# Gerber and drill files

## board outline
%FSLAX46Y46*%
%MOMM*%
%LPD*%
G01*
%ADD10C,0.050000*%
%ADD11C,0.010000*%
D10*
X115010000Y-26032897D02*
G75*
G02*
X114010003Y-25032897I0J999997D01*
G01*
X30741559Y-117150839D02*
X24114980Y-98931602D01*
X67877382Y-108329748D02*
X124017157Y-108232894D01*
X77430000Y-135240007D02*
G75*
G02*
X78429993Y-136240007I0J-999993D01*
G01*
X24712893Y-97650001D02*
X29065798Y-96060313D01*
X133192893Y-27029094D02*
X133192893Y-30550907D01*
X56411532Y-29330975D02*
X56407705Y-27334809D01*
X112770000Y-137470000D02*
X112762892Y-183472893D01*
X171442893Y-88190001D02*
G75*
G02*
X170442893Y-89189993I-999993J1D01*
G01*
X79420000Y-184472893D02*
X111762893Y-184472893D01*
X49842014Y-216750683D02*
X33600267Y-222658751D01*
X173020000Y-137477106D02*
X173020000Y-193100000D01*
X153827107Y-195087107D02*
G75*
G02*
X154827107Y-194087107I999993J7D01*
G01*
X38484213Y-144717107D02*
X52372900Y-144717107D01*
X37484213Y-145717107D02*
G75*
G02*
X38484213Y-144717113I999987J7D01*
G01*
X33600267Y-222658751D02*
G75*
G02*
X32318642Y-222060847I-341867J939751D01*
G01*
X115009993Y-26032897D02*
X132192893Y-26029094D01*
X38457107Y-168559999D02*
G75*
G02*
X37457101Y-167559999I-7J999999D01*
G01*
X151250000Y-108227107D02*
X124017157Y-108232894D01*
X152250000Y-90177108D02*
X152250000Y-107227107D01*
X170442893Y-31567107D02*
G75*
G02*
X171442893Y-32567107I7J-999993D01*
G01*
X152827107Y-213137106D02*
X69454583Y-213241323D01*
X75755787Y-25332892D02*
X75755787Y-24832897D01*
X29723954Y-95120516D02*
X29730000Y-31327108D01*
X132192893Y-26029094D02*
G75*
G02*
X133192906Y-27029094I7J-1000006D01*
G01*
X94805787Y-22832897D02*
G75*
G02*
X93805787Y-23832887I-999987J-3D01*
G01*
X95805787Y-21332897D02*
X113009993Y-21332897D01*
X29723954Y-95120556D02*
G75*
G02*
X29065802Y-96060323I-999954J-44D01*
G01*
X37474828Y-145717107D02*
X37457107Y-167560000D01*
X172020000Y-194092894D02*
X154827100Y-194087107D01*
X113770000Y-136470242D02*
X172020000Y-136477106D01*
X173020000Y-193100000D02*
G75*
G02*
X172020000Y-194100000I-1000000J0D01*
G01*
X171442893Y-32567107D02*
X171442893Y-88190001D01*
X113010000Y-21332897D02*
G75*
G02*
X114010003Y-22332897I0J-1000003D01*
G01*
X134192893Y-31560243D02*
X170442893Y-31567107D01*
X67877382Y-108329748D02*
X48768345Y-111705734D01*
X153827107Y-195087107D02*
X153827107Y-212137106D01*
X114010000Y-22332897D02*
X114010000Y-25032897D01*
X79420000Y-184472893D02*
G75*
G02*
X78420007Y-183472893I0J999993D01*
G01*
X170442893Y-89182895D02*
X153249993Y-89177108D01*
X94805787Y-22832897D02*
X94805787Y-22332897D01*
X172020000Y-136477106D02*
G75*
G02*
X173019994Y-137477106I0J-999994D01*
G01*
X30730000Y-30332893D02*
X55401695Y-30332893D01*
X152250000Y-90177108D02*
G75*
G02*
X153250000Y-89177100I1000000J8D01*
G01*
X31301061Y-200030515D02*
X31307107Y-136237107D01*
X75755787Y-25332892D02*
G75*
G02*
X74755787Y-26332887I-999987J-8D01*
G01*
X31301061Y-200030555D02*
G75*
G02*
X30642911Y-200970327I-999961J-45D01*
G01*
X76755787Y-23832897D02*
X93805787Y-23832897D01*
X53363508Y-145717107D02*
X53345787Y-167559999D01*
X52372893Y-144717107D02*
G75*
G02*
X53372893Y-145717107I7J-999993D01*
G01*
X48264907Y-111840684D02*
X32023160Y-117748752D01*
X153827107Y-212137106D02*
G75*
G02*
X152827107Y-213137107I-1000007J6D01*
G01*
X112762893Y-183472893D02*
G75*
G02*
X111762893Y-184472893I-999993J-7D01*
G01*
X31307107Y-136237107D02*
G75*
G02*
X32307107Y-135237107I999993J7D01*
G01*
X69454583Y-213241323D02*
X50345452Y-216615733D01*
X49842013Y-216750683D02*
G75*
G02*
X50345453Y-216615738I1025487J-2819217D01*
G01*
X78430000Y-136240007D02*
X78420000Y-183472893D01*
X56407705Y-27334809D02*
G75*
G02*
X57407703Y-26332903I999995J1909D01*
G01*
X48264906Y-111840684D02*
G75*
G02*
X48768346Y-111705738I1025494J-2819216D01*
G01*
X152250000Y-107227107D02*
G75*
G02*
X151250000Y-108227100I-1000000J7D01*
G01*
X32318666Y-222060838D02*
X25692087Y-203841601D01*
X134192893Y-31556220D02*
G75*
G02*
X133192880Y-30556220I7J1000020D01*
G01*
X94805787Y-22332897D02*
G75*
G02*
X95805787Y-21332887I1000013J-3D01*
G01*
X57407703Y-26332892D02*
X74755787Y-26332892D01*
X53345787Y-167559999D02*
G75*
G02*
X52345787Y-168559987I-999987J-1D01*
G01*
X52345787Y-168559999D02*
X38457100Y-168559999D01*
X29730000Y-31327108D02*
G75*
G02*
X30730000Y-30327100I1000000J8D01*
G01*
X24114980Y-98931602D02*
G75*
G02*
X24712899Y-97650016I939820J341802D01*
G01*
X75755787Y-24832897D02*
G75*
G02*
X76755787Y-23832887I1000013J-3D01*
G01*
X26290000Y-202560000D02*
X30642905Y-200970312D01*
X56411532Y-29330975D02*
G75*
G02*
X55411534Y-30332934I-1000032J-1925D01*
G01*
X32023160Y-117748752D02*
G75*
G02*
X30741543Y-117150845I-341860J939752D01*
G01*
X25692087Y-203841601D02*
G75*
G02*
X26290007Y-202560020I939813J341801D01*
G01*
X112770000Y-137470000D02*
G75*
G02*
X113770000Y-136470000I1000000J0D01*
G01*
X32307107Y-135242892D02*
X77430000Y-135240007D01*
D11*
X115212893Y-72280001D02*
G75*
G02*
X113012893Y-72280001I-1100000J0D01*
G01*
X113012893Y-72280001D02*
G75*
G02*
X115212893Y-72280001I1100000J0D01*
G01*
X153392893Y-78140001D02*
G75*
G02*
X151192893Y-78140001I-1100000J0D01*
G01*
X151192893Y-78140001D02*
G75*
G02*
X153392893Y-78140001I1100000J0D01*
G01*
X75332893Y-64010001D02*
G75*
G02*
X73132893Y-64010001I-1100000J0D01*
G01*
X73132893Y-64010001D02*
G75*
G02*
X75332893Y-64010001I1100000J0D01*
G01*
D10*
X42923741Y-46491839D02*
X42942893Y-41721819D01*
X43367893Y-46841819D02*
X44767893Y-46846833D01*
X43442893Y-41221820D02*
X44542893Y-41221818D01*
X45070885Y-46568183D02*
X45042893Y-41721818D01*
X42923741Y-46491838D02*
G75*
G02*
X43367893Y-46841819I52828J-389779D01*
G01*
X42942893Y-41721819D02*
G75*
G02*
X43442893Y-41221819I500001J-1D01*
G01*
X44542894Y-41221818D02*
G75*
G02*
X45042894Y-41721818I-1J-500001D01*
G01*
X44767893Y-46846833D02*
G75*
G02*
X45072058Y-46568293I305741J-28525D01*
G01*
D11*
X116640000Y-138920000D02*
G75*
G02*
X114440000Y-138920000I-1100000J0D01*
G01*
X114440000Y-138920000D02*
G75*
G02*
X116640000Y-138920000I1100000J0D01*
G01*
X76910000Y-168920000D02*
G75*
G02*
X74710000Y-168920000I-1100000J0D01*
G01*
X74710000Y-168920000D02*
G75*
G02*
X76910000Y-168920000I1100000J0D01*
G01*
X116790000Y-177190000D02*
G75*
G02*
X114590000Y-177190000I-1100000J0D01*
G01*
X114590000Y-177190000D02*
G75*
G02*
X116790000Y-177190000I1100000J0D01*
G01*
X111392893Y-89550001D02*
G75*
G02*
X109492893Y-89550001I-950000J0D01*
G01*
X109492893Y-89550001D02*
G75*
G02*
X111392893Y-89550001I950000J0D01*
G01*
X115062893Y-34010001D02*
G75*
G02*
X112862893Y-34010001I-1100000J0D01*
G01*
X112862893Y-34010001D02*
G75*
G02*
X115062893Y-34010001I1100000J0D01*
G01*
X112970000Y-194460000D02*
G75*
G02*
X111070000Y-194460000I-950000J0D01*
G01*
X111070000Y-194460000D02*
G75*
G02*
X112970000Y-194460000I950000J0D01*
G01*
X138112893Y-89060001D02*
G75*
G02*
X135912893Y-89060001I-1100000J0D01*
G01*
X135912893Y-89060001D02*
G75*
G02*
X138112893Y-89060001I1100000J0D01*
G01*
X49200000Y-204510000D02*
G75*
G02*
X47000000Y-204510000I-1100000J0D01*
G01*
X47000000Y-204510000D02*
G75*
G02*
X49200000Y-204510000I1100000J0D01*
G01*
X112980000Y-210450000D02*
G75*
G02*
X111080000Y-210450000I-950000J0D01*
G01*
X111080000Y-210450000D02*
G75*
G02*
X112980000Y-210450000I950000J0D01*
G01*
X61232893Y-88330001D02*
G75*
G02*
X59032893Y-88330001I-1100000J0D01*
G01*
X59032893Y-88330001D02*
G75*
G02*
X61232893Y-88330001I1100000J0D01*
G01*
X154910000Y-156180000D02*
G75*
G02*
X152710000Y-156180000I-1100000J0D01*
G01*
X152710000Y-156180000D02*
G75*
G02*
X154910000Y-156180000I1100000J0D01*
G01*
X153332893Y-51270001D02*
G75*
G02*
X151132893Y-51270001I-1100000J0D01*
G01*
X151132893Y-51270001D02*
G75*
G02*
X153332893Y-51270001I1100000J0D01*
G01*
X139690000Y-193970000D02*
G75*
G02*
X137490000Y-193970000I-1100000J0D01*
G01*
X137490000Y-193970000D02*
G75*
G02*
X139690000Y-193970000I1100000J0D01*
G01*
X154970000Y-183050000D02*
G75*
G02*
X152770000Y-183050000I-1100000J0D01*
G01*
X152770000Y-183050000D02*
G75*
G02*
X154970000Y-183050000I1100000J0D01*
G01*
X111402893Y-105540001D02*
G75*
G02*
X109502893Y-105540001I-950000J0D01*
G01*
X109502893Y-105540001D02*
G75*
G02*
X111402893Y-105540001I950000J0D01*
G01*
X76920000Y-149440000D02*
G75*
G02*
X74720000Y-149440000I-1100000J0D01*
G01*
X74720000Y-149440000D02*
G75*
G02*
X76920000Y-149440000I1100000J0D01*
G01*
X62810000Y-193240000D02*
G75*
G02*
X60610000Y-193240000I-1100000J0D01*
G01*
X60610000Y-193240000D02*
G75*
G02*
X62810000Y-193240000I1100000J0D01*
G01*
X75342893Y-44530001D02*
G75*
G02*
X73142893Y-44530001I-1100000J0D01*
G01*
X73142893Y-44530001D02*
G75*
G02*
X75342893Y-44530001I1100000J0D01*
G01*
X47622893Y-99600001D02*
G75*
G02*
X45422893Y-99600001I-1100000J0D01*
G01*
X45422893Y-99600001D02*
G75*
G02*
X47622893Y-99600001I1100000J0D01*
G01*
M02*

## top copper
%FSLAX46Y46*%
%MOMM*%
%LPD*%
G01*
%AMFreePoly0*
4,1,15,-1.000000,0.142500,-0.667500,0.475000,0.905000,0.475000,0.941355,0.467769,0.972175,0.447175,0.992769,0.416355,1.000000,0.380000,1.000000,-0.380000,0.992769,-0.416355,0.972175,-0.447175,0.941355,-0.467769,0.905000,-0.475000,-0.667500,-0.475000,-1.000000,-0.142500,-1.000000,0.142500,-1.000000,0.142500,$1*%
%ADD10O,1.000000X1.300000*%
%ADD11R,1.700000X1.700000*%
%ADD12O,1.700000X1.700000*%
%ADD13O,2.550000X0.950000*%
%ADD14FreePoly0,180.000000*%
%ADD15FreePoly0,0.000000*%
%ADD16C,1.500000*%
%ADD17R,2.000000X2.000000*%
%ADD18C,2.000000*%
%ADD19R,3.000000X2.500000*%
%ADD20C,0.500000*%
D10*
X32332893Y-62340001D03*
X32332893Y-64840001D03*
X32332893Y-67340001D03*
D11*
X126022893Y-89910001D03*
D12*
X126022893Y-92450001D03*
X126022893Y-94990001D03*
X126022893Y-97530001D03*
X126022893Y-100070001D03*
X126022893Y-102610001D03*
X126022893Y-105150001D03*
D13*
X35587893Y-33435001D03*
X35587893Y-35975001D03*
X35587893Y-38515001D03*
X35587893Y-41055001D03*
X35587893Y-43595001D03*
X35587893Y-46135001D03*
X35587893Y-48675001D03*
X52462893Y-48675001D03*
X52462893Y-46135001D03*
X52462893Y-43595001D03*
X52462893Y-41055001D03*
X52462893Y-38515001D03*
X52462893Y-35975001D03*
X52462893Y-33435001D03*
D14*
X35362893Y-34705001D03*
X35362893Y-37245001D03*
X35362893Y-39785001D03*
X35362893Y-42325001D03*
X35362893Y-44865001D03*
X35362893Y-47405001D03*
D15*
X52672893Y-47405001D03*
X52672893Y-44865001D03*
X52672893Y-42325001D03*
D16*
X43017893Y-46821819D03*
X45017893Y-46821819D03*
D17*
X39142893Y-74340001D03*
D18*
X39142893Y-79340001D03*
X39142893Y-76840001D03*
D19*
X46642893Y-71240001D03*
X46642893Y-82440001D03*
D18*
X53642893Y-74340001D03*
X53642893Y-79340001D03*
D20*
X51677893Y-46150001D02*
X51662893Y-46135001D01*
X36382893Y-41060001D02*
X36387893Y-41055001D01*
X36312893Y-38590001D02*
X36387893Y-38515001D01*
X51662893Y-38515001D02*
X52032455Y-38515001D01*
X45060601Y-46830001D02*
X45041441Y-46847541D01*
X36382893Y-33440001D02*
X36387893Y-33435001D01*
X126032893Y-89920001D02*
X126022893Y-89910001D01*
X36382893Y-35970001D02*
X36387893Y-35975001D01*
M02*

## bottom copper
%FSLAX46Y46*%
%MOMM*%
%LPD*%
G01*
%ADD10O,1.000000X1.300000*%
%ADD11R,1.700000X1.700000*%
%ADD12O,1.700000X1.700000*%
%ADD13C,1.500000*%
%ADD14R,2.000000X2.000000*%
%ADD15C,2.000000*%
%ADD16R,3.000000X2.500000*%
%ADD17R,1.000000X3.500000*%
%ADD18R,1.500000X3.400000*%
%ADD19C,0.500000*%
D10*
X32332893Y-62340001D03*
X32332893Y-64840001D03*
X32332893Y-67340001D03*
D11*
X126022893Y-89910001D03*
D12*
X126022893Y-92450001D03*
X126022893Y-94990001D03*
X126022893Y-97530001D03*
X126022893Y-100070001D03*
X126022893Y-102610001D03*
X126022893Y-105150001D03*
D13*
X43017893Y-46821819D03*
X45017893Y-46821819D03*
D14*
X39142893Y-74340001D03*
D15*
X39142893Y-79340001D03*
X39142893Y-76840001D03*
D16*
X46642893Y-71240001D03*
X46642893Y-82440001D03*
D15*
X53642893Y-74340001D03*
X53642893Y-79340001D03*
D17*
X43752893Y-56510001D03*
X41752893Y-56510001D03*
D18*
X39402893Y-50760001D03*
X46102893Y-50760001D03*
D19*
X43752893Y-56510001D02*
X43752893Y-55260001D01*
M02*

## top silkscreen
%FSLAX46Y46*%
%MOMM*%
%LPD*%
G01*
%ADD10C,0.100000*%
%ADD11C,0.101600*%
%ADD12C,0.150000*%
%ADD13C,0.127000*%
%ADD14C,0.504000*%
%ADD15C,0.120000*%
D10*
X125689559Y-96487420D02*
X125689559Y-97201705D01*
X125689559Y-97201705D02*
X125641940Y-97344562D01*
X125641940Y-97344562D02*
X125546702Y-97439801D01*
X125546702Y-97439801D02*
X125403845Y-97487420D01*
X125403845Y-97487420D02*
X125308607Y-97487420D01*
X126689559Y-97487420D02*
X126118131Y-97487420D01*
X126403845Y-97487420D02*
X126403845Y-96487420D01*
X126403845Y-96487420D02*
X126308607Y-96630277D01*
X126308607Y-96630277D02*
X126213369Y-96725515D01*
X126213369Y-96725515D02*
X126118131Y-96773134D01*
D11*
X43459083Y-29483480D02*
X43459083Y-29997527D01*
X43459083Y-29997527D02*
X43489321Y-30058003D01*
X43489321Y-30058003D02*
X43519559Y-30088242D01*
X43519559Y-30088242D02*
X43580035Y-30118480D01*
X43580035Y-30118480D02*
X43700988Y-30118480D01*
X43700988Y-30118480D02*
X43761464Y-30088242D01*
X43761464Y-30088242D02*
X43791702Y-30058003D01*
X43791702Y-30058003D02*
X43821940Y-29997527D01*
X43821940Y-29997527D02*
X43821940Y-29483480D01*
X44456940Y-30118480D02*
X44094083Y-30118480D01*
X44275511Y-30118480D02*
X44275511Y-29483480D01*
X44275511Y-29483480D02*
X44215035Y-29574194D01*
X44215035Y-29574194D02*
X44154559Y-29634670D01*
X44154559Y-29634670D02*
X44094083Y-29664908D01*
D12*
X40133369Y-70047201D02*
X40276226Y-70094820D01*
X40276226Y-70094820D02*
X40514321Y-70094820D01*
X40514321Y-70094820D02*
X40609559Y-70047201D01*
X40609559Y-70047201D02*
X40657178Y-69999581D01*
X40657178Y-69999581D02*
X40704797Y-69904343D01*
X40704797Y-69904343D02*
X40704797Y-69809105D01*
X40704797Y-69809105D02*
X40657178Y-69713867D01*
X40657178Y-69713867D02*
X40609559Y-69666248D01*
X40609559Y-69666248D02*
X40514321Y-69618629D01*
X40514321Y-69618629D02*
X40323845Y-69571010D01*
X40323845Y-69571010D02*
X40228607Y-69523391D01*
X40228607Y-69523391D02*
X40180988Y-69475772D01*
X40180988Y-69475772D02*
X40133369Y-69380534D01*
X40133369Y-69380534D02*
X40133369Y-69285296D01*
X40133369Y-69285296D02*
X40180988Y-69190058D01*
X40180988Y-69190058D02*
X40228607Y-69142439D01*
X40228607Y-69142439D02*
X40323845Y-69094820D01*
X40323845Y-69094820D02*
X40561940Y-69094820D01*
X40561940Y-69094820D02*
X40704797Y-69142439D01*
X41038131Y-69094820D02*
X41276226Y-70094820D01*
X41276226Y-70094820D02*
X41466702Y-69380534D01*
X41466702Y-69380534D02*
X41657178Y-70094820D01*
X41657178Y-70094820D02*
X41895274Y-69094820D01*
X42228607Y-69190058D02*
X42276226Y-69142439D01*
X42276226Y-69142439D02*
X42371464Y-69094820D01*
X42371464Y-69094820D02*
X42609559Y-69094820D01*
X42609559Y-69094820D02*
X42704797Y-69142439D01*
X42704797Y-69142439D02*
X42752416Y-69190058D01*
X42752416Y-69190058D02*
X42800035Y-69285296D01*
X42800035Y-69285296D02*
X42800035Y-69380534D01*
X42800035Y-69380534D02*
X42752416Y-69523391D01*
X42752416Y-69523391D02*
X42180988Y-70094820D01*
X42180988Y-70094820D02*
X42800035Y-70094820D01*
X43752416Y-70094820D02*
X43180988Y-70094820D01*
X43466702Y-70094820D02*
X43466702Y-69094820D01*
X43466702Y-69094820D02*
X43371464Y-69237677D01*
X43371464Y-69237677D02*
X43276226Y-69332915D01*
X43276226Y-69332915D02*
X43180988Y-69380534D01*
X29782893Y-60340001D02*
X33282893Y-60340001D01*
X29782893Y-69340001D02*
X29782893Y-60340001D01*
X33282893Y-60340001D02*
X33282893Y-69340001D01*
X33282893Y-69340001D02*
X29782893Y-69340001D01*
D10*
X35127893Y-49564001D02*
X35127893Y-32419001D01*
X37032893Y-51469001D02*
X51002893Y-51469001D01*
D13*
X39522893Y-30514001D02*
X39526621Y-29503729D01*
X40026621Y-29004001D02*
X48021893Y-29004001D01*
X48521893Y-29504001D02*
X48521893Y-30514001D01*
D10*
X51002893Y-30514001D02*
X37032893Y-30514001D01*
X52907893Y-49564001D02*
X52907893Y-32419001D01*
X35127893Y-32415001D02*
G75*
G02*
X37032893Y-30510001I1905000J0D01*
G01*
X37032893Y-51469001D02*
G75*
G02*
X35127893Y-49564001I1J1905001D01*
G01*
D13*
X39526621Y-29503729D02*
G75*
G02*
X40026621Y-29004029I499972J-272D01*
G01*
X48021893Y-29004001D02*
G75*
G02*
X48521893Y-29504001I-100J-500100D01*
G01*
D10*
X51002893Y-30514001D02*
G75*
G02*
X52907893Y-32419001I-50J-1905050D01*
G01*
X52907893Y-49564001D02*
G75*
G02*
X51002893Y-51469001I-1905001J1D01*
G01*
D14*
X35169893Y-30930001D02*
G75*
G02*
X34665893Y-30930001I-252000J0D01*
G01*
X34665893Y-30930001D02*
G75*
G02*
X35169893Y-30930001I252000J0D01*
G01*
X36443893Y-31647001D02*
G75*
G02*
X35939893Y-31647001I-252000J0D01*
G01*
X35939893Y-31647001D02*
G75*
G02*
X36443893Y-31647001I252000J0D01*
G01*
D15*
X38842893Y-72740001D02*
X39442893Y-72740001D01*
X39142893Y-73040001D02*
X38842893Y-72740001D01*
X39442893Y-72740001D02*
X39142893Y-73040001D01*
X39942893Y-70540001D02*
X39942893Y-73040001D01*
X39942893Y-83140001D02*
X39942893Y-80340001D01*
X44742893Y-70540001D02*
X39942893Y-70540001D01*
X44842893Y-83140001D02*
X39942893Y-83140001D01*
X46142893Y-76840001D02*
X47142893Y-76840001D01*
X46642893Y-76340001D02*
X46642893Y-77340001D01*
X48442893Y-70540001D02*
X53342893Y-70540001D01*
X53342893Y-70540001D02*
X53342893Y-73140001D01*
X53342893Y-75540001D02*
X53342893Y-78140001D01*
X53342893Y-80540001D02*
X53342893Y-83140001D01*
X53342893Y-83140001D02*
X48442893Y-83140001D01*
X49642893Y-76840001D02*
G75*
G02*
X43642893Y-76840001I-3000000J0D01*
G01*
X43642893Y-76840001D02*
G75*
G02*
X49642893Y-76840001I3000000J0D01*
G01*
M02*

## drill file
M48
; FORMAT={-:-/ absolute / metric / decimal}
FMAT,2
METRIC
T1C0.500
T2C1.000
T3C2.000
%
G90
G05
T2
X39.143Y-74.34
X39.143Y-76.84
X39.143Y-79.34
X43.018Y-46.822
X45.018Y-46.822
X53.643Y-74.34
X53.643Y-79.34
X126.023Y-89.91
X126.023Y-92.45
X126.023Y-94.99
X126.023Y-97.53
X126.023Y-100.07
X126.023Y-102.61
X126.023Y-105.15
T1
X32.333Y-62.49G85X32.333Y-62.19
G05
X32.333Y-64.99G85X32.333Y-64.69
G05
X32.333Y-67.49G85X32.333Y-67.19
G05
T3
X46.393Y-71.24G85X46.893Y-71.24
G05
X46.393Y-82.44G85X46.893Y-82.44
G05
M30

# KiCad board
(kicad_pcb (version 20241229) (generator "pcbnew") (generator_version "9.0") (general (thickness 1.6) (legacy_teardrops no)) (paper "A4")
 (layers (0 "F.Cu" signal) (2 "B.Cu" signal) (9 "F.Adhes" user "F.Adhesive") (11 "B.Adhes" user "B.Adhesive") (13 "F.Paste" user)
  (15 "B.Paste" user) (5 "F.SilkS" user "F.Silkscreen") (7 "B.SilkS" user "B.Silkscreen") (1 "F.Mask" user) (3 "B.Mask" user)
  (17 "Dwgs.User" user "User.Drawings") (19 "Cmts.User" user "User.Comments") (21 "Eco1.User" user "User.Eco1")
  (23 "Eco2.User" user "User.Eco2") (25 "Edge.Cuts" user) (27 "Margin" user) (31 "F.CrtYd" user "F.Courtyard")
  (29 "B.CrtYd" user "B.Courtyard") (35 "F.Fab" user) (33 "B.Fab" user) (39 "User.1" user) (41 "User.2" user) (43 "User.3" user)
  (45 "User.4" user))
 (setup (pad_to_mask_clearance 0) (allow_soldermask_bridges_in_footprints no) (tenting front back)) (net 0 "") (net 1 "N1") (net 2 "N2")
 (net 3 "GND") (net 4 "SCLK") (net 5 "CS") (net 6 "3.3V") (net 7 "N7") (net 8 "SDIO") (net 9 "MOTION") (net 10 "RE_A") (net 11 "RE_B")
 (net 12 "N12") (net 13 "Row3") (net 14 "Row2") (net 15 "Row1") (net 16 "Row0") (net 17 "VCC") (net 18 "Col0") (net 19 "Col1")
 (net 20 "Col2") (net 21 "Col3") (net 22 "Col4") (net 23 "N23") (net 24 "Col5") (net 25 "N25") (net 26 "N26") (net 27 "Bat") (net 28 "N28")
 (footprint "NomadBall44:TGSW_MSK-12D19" (layer "F.Cu") (at 31.282893 64.840001 90)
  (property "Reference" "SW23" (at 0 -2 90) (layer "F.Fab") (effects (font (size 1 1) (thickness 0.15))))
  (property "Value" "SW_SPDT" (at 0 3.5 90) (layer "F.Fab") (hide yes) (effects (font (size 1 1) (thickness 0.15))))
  (fp_line (start 4.5 -1.5) (end 4.5 2) (stroke (width 0.15) (type solid)) (layer "F.SilkS"))
  (fp_line (start -4.5 -1.5) (end 4.5 -1.5) (stroke (width 0.15) (type solid)) (layer "F.SilkS"))
  (fp_line (start 4.5 2) (end -4.5 2) (stroke (width 0.15) (type solid)) (layer "F.SilkS"))
  (fp_line (start -4.5 2) (end -4.5 -1.5) (stroke (width 0.15) (type solid)) (layer "F.SilkS"))
  (pad "1" thru_hole oval (at 2.5 1.05 90) (size 1.3 1) (drill oval 0.8 0.5) (layers "*.Cu" "*.Mask") (remove_unused_layers no) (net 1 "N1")
   (clearance 0.15))
  (pad "2" thru_hole oval (at 0 1.05 90) (size 1.3 1) (drill oval 0.8 0.5) (layers "*.Cu" "*.Mask") (remove_unused_layers no) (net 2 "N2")
   (clearance 0.15))
  (pad "3" thru_hole oval (at -2.5 1.05 90) (size 1.3 1) (drill oval 0.8 0.5) (layers "*.Cu" "*.Mask") (remove_unused_layers no)
   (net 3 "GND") (clearance 0.15)))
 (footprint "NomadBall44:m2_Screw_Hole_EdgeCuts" (layer "F.Cu") (at 114.112893 72.280001)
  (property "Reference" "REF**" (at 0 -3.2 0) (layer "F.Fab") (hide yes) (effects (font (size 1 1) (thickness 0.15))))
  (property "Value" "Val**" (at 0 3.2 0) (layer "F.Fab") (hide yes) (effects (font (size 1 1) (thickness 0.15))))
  (fp_circle (center 0 0) (end 1.1 0) (stroke (width 0.01) (type solid)) (fill no) (layer "Edge.Cuts")))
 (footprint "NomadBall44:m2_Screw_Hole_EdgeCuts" (layer "F.Cu") (at 152.292893 78.140001)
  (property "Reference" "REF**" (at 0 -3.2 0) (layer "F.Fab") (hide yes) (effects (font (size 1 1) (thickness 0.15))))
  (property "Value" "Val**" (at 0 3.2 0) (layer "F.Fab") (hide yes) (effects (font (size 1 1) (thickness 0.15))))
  (fp_circle (center 0 0) (end 1.1 0) (stroke (width 0.01) (type solid)) (fill no) (layer "Edge.Cuts")))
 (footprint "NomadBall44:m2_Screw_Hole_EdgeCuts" (layer "F.Cu") (at 74.232893 64.010001)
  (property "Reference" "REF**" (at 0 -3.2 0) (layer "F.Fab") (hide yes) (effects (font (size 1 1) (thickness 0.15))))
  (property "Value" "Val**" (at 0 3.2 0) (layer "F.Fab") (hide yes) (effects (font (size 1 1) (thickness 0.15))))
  (fp_circle (center 0 0) (end 1.1 0) (stroke (width 0.01) (type solid)) (fill no) (layer "Edge.Cuts")))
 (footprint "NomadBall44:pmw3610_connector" (layer "F.Cu") (at 126.022893 97.530001)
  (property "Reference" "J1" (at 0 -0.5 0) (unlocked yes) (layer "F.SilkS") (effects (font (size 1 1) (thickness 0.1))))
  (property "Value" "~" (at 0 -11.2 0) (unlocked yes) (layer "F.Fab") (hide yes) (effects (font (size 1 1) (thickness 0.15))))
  (pad "1" thru_hole rect (at 0 -7.62) (size 1.7 1.7) (drill 1) (layers "*.Cu" "*.Mask") (remove_unused_layers no) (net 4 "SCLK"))
  (pad "2" thru_hole oval (at 0 -5.08) (size 1.7 1.7) (drill 1) (layers "*.Cu" "*.Mask") (remove_unused_layers no) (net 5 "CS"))
  (pad "3" thru_hole oval (at 0 -2.54) (size 1.7 1.7) (drill 1) (layers "*.Cu" "*.Mask") (remove_unused_layers no) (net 3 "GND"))
  (pad "4" thru_hole oval (at 0 0) (size 1.7 1.7) (drill 1) (layers "*.Cu" "*.Mask") (remove_unused_layers no) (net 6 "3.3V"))
  (pad "5" thru_hole oval (at 0 2.54) (size 1.7 1.7) (drill 1) (layers "*.Cu" "*.Mask") (remove_unused_layers no) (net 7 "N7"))
  (pad "6" thru_hole oval (at 0 5.08) (size 1.7 1.7) (drill 1) (layers "*.Cu" "*.Mask") (remove_unused_layers no) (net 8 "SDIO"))
  (pad "7" thru_hole oval (at 0 7.62) (size 1.7 1.7) (drill 1) (layers "*.Cu" "*.Mask") (remove_unused_layers no) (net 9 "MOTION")))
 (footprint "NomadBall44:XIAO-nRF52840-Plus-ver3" (layer "F.Cu") (at 42.617893 40.955001 90)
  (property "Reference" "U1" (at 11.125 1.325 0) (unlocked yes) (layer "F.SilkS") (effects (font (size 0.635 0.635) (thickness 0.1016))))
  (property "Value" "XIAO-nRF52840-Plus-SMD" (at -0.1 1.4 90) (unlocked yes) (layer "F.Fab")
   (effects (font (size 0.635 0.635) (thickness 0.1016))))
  (fp_line (start -8.609 -7.49) (end 8.536 -7.49) (stroke (width 0.1) (type solid)) (layer "F.SilkS"))
  (fp_line (start -10.514 -5.585) (end -10.514 8.385) (stroke (width 0.1) (type solid)) (layer "F.SilkS"))
  (fp_line (start 10.441 -3.095) (end 11.451272 -3.091272) (stroke (width 0.127) (type solid)) (layer "F.SilkS"))
  (fp_line (start 11.951 -2.591272) (end 11.951 5.404) (stroke (width 0.127) (type solid)) (layer "F.SilkS"))
  (fp_line (start 11.451 5.904) (end 10.441 5.904) (stroke (width 0.127) (type solid)) (layer "F.SilkS"))
  (fp_line (start 10.441 8.385) (end 10.441 -5.585) (stroke (width 0.1) (type solid)) (layer "F.SilkS"))
  (fp_line (start -8.609 10.29) (end 8.536 10.29) (stroke (width 0.1) (type solid)) (layer "F.SilkS"))
  (fp_arc (start 8.54 -7.49) (mid 9.887038 -6.932038) (end 10.445 -5.585) (stroke (width 0.1) (type solid)) (layer "F.SilkS"))
  (fp_arc (start -10.514 -5.585) (mid -9.956038 -6.932038) (end -8.609 -7.49) (stroke (width 0.1) (type solid)) (layer "F.SilkS"))
  (fp_arc (start 11.451272 -3.091272) (mid 11.80464 -2.944728) (end 11.951 -2.591272) (stroke (width 0.127) (type default))
   (layer "F.SilkS"))
  (fp_arc (start 11.951 5.404) (mid 11.804524 5.757524) (end 11.451 5.904) (stroke (width 0.127) (type default)) (layer "F.SilkS"))
  (fp_arc (start 10.441 8.385) (mid 9.883024 9.732024) (end 8.536 10.29) (stroke (width 0.1) (type solid)) (layer "F.SilkS"))
  (fp_arc (start -8.609 10.29) (mid -9.956038 9.732038) (end -10.514 8.385) (stroke (width 0.1) (type solid)) (layer "F.SilkS"))
  (fp_circle (center 10.025 -7.7) (end 10.279 -7.7) (stroke (width 0.5) (type solid)) (fill yes) (layer "F.SilkS"))
  (fp_circle (center 9.308 -6.426) (end 9.562 -6.426) (stroke (width 0.5) (type solid)) (fill yes) (layer "F.SilkS"))
  (fp_line (start -5.536838 0.305848) (end -0.766818 0.325) (stroke (width 0.05) (type default)) (layer "Edge.Cuts"))
  (fp_line (start -5.886818 0.75) (end -5.891832 2.15) (stroke (width 0.05) (type default)) (layer "Edge.Cuts"))
  (fp_line (start -0.266819 0.825) (end -0.266817 1.925) (stroke (width 0.05) (type default)) (layer "Edge.Cuts"))
  (fp_line (start -5.613182 2.452992) (end -0.766817 2.425) (stroke (width 0.05) (type default)) (layer "Edge.Cuts"))
  (fp_arc (start -5.536837 0.305848) (mid -5.617663 0.602123) (end -5.886818 0.75) (stroke (width 0.05) (type default)) (layer "Edge.Cuts"))
  (fp_arc (start -0.766818 0.325) (mid -0.413265 0.471447) (end -0.266818 0.825) (stroke (width 0.05) (type default)) (layer "Edge.Cuts"))
  (fp_arc (start -0.266817 1.925001) (mid -0.413264 2.278554) (end -0.766817 2.425001) (stroke (width 0.05) (type default))
   (layer "Edge.Cuts"))
  (fp_arc (start -5.891832 2.15) (mid -5.693897 2.24836) (end -5.613293 2.454165) (stroke (width 0.05) (type default)) (layer "Edge.Cuts"))
  (pad "1" smd oval (at 7.52 -6.23) (size 2.55 0.95) (drill (offset -0.8 0)) (layers "F.Cu" "F.Mask" "F.Paste") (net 8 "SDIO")
   (thermal_bridge_angle 45))
  (pad "2" smd oval (at 4.98 -6.23) (size 2.55 0.95) (drill (offset -0.8 0)) (layers "F.Cu" "F.Mask" "F.Paste") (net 4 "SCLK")
   (thermal_bridge_angle 45))
  (pad "3" smd oval (at 2.44 -6.23) (size 2.55 0.95) (drill (offset -0.8 0)) (layers "F.Cu" "F.Mask" "F.Paste") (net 5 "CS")
   (thermal_bridge_angle 45))
  (pad "4" smd oval (at -0.1 -6.23) (size 2.55 0.95) (drill (offset -0.8 0)) (layers "F.Cu" "F.Mask" "F.Paste") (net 9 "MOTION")
   (thermal_bridge_angle 45))
  (pad "5" smd oval (at -2.64 -6.23) (size 2.55 0.95) (drill (offset -0.8 0)) (layers "F.Cu" "F.Mask" "F.Paste") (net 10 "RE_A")
   (thermal_bridge_angle 45))
  (pad "6" smd oval (at -5.18 -6.23) (size 2.55 0.95) (drill (offset -0.8 0)) (layers "F.Cu" "F.Mask" "F.Paste") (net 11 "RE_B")
   (thermal_bridge_angle 45))
  (pad "7" smd oval (at -7.72 -6.23) (size 2.55 0.95) (drill (offset -0.8 0)) (layers "F.Cu" "F.Mask" "F.Paste") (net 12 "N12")
   (thermal_bridge_angle 45))
  (pad "8" smd oval (at -7.72 9.045) (size 2.55 0.95) (drill (offset 0.8 0)) (layers "F.Cu" "F.Mask" "F.Paste") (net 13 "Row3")
   (thermal_bridge_angle 45))
  (pad "9" smd oval (at -5.18 9.045) (size 2.55 0.95) (drill (offset 0.8 0)) (layers "F.Cu" "F.Mask" "F.Paste") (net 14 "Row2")
   (thermal_bridge_angle 45))
  (pad "10" smd oval (at -2.64 9.045) (size 2.55 0.95) (drill (offset 0.8 0)) (layers "F.Cu" "F.Mask" "F.Paste") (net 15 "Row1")
   (thermal_bridge_angle 45))
  (pad "11" smd oval (at -0.1 9.045) (size 2.55 0.95) (drill (offset 0.8 0)) (layers "F.Cu" "F.Mask" "F.Paste") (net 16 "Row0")
   (thermal_bridge_angle 45))
  (pad "12" smd oval (at 2.44 9.045) (size 2.55 0.95) (drill (offset 0.8 0)) (layers "F.Cu" "F.Mask" "F.Paste") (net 6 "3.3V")
   (thermal_bridge_angle 45))
  (pad "13" smd oval (at 4.98 9.045) (size 2.55 0.95) (drill (offset 0.8 0)) (layers "F.Cu" "F.Mask" "F.Paste") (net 3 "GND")
   (thermal_bridge_angle 45))
  (pad "14" smd oval (at 7.52 9.045) (size 2.55 0.95) (drill (offset 0.8 0)) (layers "F.Cu" "F.Mask" "F.Paste") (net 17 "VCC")
   (thermal_bridge_angle 45))
  (pad "15" smd roundrect (at 6.25 -7.255 180) (size 2 0.95) (layers "F.Cu" "F.Mask" "F.Paste") (roundrect_rratio 0.1) (chamfer_ratio 0.35)
   (chamfer top_left bottom_left) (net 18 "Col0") (thermal_bridge_angle 45))
  (pad "16" smd roundrect (at 3.71 -7.255 180) (size 2 0.95) (layers "F.Cu" "F.Mask" "F.Paste") (roundrect_rratio 0.1) (chamfer_ratio 0.35)
   (chamfer top_left bottom_left) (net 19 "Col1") (thermal_bridge_angle 45))
  (pad "17" smd roundrect (at 1.17 -7.255 180) (size 2 0.95) (layers "F.Cu" "F.Mask" "F.Paste") (roundrect_rratio 0.1) (chamfer_ratio 0.35)
   (chamfer top_left bottom_left) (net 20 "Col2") (thermal_bridge_angle 45))
  (pad "18" smd roundrect (at -1.37 -7.255 180) (size 2 0.95) (layers "F.Cu" "F.Mask" "F.Paste") (roundrect_rratio 0.1) (chamfer_ratio 0.35)
   (chamfer top_left bottom_left) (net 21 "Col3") (thermal_bridge_angle 45))
  (pad "19" smd roundrect (at -3.91 -7.255 180) (size 2 0.95) (layers "F.Cu" "F.Mask" "F.Paste") (roundrect_rratio 0.1) (chamfer_ratio 0.35)
   (chamfer top_left bottom_left) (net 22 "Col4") (thermal_bridge_angle 45))
  (pad "20" smd roundrect (at -6.45 -7.255 180) (size 2 0.95) (layers "F.Cu" "F.Mask" "F.Paste") (roundrect_rratio 0.1) (chamfer_ratio 0.35)
   (chamfer top_left bottom_left) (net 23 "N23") (thermal_bridge_angle 45))
  (pad "21" smd roundrect (at -6.45 10.055) (size 2 0.95) (layers "F.Cu" "F.Mask" "F.Paste") (roundrect_rratio 0.1) (chamfer_ratio 0.35)
   (chamfer top_left bottom_left) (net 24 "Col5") (thermal_bridge_angle 45))
  (pad "22" smd roundrect (at -3.91 10.055) (size 2 0.95) (layers "F.Cu" "F.Mask" "F.Paste") (roundrect_rratio 0.1) (chamfer_ratio 0.35)
   (chamfer top_left bottom_left) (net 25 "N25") (thermal_bridge_angle 45))
  (pad "23" smd roundrect (at -1.37 10.055) (size 2 0.95) (layers "F.Cu" "F.Mask" "F.Paste") (roundrect_rratio 0.1) (chamfer_ratio 0.35)
   (chamfer top_left bottom_left) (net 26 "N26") (thermal_bridge_angle 45))
  (pad "32" thru_hole circle (at -5.866818 0.4 90) (size 1.5 1.5) (drill 1) (layers "*.Cu" "*.Mask") (remove_unused_layers no)
   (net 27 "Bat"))
  (pad "33" thru_hole circle (at -5.866818 2.4 90) (size 1.5 1.5) (drill 1) (layers "*.Cu" "*.Mask") (remove_unused_layers no) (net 3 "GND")))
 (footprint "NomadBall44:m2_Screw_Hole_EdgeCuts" (layer "F.Cu") (at 115.54 138.92)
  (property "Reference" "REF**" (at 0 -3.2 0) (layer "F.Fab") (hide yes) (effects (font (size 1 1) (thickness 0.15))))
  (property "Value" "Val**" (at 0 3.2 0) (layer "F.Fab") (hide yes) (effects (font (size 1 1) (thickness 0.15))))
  (fp_circle (center 0 0) (end 1.1 0) (stroke (width 0.01) (type solid)) (fill no) (layer "Edge.Cuts")))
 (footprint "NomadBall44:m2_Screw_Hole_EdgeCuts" (layer "F.Cu") (at 75.81 168.92)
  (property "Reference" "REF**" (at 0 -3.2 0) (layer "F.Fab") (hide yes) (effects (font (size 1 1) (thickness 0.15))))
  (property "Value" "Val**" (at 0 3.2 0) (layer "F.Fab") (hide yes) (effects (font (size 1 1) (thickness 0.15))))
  (fp_circle (center 0 0) (end 1.1 0) (stroke (width 0.01) (type solid)) (fill no) (layer "Edge.Cuts")))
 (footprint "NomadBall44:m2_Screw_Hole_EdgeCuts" (layer "F.Cu") (at 115.69 177.19)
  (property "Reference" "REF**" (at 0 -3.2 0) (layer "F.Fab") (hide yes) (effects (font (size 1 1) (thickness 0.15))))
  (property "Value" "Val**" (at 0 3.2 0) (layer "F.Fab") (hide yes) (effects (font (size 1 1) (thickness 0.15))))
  (fp_circle (center 0 0) (end 1.1 0) (stroke (width 0.01) (type solid)) (fill no) (layer "Edge.Cuts")))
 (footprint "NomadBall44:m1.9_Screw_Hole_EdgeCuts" (layer "F.Cu") (at 110.442893 89.550001)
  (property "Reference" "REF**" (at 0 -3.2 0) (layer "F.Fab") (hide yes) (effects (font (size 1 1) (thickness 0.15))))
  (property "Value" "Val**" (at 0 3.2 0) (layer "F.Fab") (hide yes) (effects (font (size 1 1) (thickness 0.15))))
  (fp_circle (center 0 0) (end 0.95 0) (stroke (width 0.01) (type solid)) (fill no) (layer "Edge.Cuts")))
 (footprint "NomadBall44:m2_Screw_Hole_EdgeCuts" (layer "F.Cu") (at 113.962893 34.010001)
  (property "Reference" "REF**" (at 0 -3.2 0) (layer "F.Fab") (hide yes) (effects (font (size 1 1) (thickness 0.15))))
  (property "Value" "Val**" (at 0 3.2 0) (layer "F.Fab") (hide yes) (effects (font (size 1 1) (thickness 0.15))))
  (fp_circle (center 0 0) (end 1.1 0) (stroke (width 0.01) (type solid)) (fill no) (layer "Edge.Cuts")))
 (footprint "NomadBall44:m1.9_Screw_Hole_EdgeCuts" (layer "F.Cu") (at 112.02 194.46)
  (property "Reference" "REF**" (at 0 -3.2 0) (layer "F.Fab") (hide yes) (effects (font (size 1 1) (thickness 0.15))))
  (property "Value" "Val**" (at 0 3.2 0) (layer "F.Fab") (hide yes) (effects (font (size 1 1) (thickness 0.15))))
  (fp_circle (center 0 0) (end 0.95 0) (stroke (width 0.01) (type solid)) (fill no) (layer "Edge.Cuts")))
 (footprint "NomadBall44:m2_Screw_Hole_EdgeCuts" (layer "F.Cu") (at 137.012893 89.060001)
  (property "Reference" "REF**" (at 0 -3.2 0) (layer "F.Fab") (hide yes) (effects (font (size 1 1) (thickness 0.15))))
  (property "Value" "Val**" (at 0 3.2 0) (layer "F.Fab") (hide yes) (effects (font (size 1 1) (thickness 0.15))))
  (fp_circle (center 0 0) (end 1.1 0) (stroke (width 0.01) (type solid)) (fill no) (layer "Edge.Cuts")))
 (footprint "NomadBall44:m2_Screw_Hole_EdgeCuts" (layer "F.Cu") (at 48.1 204.51)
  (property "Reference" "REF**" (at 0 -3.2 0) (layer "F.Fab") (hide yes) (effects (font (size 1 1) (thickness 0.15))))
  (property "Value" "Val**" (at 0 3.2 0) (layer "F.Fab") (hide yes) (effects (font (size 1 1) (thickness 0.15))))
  (fp_circle (center 0 0) (end 1.1 0) (stroke (width 0.01) (type solid)) (fill no) (layer "Edge.Cuts")))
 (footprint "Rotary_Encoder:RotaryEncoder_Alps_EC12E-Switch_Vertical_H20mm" (layer "F.Cu") (at 39.142893 74.340001)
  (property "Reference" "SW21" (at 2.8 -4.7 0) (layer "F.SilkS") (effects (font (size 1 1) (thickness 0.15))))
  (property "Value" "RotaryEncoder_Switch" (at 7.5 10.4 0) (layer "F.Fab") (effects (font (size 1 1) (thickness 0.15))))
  (fp_line (start -0.3 -1.6) (end 0.3 -1.6) (stroke (width 0.12) (type solid)) (layer "F.SilkS"))
  (fp_line (start 0 -1.3) (end -0.3 -1.6) (stroke (width 0.12) (type solid)) (layer "F.SilkS"))
  (fp_line (start 0.3 -1.6) (end 0 -1.3) (stroke (width 0.12) (type solid)) (layer "F.SilkS"))
  (fp_line (start 0.8 -3.8) (end 0.8 -1.3) (stroke (width 0.12) (type solid)) (layer "F.SilkS"))
  (fp_line (start 0.8 8.8) (end 0.8 6) (stroke (width 0.12) (type solid)) (layer "F.SilkS"))
  (fp_line (start 5.6 -3.8) (end 0.8 -3.8) (stroke (width 0.12) (type solid)) (layer "F.SilkS"))
  (fp_line (start 5.7 8.8) (end 0.8 8.8) (stroke (width 0.12) (type solid)) (layer "F.SilkS"))
  (fp_line (start 7 2.5) (end 8 2.5) (stroke (width 0.12) (type solid)) (layer "F.SilkS"))
  (fp_line (start 7.5 2) (end 7.5 3) (stroke (width 0.12) (type solid)) (layer "F.SilkS"))
  (fp_line (start 9.3 -3.8) (end 14.2 -3.8) (stroke (width 0.12) (type solid)) (layer "F.SilkS"))
  (fp_line (start 14.2 -3.8) (end 14.2 -1.2) (stroke (width 0.12) (type solid)) (layer "F.SilkS"))
  (fp_line (start 14.2 1.2) (end 14.2 3.8) (stroke (width 0.12) (type solid)) (layer "F.SilkS"))
  (fp_line (start 14.2 6.2) (end 14.2 8.8) (stroke (width 0.12) (type solid)) (layer "F.SilkS"))
  (fp_line (start 14.2 8.8) (end 9.3 8.8) (stroke (width 0.12) (type solid)) (layer "F.SilkS"))
  (fp_circle (center 7.5 2.5) (end 10.5 2.5) (stroke (width 0.12) (type solid)) (fill no) (layer "F.SilkS"))
  (pad "A" thru_hole rect (at 0 0) (size 2 2) (drill 1) (layers "*.Cu" "*.Mask") (remove_unused_layers no) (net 10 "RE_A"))
  (pad "B" thru_hole circle (at 0 5) (size 2 2) (drill 1) (layers "*.Cu" "*.Mask") (remove_unused_layers no) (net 11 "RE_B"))
  (pad "C" thru_hole circle (at 0 2.5) (size 2 2) (drill 1) (layers "*.Cu" "*.Mask") (remove_unused_layers no) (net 3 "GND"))
  (pad "MP" thru_hole rect (at 7.5 -3.1) (size 3 2.5) (drill oval 2.5 2) (layers "*.Cu" "*.Mask") (remove_unused_layers no))
  (pad "MP" thru_hole rect (at 7.5 8.1) (size 3 2.5) (drill oval 2.5 2) (layers "*.Cu" "*.Mask") (remove_unused_layers no))
  (pad "S1" thru_hole circle (at 14.5 0) (size 2 2) (drill 1) (layers "*.Cu" "*.Mask") (remove_unused_layers no) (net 20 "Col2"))
  (pad "S2" thru_hole circle (at 14.5 5) (size 2 2) (drill 1) (layers "*.Cu" "*.Mask") (remove_unused_layers no) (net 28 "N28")))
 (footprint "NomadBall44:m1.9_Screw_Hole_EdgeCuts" (layer "F.Cu") (at 112.03 210.45)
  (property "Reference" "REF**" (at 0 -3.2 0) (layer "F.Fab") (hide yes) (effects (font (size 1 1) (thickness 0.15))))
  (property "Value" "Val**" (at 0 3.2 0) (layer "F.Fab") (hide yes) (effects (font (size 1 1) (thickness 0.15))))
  (fp_circle (center 0 0) (end 0.95 0) (stroke (width 0.01) (type solid)) (fill no) (layer "Edge.Cuts")))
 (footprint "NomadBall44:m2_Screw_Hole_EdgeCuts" (layer "F.Cu") (at 60.132893 88.330001)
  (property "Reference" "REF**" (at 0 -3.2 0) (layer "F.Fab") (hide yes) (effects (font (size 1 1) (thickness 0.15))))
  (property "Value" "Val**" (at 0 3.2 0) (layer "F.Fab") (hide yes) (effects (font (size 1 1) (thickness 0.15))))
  (fp_circle (center 0 0) (end 1.1 0) (stroke (width 0.01) (type solid)) (fill no) (layer "Edge.Cuts")))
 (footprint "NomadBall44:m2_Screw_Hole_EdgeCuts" (layer "F.Cu") (at 153.81 156.18)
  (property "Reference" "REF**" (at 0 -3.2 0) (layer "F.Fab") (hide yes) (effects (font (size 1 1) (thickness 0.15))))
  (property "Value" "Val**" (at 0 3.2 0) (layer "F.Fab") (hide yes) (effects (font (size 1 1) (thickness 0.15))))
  (fp_circle (center 0 0) (end 1.1 0) (stroke (width 0.01) (type solid)) (fill no) (layer "Edge.Cuts")))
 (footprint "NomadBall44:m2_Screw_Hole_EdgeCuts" (layer "F.Cu") (at 152.232893 51.270001)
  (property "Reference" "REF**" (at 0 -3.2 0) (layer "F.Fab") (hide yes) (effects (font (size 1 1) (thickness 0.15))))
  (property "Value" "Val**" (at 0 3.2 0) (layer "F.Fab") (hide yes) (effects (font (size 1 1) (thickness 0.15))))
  (fp_circle (center 0 0) (end 1.1 0) (stroke (width 0.01) (type solid)) (fill no) (layer "Edge.Cuts")))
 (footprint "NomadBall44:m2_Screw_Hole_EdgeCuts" (layer "F.Cu") (at 138.59 193.97)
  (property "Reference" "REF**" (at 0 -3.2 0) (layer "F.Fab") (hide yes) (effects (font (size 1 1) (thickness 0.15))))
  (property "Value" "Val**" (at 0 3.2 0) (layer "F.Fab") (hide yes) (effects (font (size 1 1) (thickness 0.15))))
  (fp_circle (center 0 0) (end 1.1 0) (stroke (width 0.01) (type solid)) (fill no) (layer "Edge.Cuts")))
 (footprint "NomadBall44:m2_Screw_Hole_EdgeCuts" (layer "F.Cu") (at 153.87 183.05)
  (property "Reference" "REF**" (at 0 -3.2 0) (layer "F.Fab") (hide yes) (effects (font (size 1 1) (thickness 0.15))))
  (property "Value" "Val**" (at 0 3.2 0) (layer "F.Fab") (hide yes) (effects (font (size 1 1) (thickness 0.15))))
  (fp_circle (center 0 0) (end 1.1 0) (stroke (width 0.01) (type solid)) (fill no) (layer "Edge.Cuts")))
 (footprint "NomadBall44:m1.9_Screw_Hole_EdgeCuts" (layer "F.Cu") (at 110.452893 105.540001)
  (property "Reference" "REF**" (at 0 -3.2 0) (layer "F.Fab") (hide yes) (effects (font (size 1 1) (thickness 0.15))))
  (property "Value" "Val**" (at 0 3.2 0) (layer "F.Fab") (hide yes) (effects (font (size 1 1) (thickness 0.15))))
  (fp_circle (center 0 0) (end 0.95 0) (stroke (width 0.01) (type solid)) (fill no) (layer "Edge.Cuts")))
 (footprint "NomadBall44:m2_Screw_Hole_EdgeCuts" (layer "F.Cu") (at 75.82 149.44)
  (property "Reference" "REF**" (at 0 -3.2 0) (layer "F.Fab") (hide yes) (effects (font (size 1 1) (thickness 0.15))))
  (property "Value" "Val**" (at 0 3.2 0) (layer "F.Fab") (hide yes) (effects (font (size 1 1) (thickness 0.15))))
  (fp_circle (center 0 0) (end 1.1 0) (stroke (width 0.01) (type solid)) (fill no) (layer "Edge.Cuts")))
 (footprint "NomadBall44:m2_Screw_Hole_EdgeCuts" (layer "F.Cu") (at 61.71 193.24)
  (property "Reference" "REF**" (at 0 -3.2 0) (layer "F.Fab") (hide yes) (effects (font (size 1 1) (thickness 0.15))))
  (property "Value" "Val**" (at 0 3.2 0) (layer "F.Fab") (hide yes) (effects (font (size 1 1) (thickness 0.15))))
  (fp_circle (center 0 0) (end 1.1 0) (stroke (width 0.01) (type solid)) (fill no) (layer "Edge.Cuts")))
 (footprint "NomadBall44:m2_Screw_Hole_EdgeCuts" (layer "F.Cu") (at 74.242893 44.530001)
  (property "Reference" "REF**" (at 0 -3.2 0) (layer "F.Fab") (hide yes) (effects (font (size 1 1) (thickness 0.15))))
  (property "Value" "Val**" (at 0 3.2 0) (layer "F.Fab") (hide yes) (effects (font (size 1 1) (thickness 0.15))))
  (fp_circle (center 0 0) (end 1.1 0) (stroke (width 0.01) (type solid)) (fill no) (layer "Edge.Cuts")))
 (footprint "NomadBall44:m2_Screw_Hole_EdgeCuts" (layer "F.Cu") (at 46.522893 99.600001)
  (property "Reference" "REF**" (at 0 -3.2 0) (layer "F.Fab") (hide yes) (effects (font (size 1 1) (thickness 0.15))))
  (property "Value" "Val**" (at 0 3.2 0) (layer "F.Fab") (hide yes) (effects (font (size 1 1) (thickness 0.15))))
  (fp_circle (center 0 0) (end 1.1 0) (stroke (width 0.01) (type solid)) (fill no) (layer "Edge.Cuts")))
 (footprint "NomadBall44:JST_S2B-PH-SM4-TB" (layer "B.Cu") (at 42.752893 56.510001 180)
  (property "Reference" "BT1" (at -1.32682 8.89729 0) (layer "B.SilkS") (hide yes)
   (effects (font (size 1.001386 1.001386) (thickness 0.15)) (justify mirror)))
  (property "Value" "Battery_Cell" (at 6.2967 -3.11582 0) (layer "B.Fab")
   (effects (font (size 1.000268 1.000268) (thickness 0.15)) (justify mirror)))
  (pad "1" smd rect (at -1 0 180) (size 1 3.5) (layers "B.Cu" "B.Mask" "B.Paste") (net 27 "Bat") (solder_mask_margin 0.102))
  (pad "2" smd rect (at 1 0 180) (size 1 3.5) (layers "B.Cu" "B.Mask" "B.Paste") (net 2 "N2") (solder_mask_margin 0.102))
  (pad "P1" smd rect (at 3.35 5.75 180) (size 1.5 3.4) (layers "B.Cu" "B.Mask" "B.Paste") (solder_mask_margin 0.102))
  (pad "P2" smd rect (at -3.35 5.75 180) (size 1.5 3.4) (layers "B.Cu" "B.Mask" "B.Paste") (solder_mask_margin 0.102)))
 (gr_arc (start 115.01 26.032897) (mid 114.302893 25.740004) (end 114.01 25.032897) (stroke (width 0.05) (type solid)) (layer "Edge.Cuts"))
 (gr_line (start 30.741559 117.150839) (end 24.11498 98.931602) (stroke (width 0.05) (type solid)) (layer "Edge.Cuts"))
 (gr_line (start 67.877382 108.329748) (end 124.017157 108.232894) (stroke (width 0.05) (type default)) (layer "Edge.Cuts"))
 (gr_arc (start 77.43 135.240007) (mid 78.137107 135.5329) (end 78.43 136.240007) (stroke (width 0.05) (type solid)) (layer "Edge.Cuts"))
 (gr_line (start 24.712893 97.650001) (end 29.065798 96.060313) (stroke (width 0.05) (type solid)) (layer "Edge.Cuts"))
 (gr_line (start 133.192893 27.029094) (end 133.192893 30.550907) (stroke (width 0.05) (type solid)) (layer "Edge.Cuts"))
 (gr_line (start 56.411532 29.330975) (end 56.407705 27.334809) (stroke (width 0.05) (type solid)) (layer "Edge.Cuts"))
 (gr_line (start 112.77 137.47) (end 112.762892 183.472893) (stroke (width 0.05) (type default)) (layer "Edge.Cuts"))
 (gr_arc (start 171.442893 88.190001) (mid 171.15 88.897108) (end 170.442893 89.190001) (stroke (width 0.05) (type solid))
  (layer "Edge.Cuts"))
 (gr_line (start 79.42 184.472893) (end 111.762893 184.472893) (stroke (width 0.05) (type default)) (layer "Edge.Cuts"))
 (gr_line (start 49.842014 216.750683) (end 33.600267 222.658751) (stroke (width 0.05) (type solid)) (layer "Edge.Cuts"))
 (gr_line (start 173.02 137.477106) (end 173.02 193.1) (stroke (width 0.05) (type solid)) (layer "Edge.Cuts"))
 (gr_arc (start 153.827107 195.087107) (mid 154.12 194.38) (end 154.827107 194.087107) (stroke (width 0.05) (type solid))
  (layer "Edge.Cuts"))
 (gr_line (start 38.484213 144.717107) (end 52.3729 144.717107) (stroke (width 0.05) (type default)) (layer "Edge.Cuts"))
 (gr_arc (start 37.484213 145.717107) (mid 37.777106 145.01) (end 38.484213 144.717107) (stroke (width 0.05) (type solid))
  (layer "Edge.Cuts"))
 (gr_arc (start 33.600267 222.658751) (mid 32.835635 222.625223) (end 32.318666 222.060838) (stroke (width 0.05) (type solid))
  (layer "Edge.Cuts"))
 (gr_line (start 115.009993 26.032897) (end 132.192893 26.029094) (stroke (width 0.05) (type solid)) (layer "Edge.Cuts"))
 (gr_arc (start 38.457107 168.559999) (mid 37.75 168.267106) (end 37.457107 167.559999) (stroke (width 0.05) (type solid))
  (layer "Edge.Cuts"))
 (gr_line (start 151.25 108.227107) (end 124.017157 108.232894) (stroke (width 0.05) (type solid)) (layer "Edge.Cuts"))
 (gr_line (start 152.25 90.177108) (end 152.25 107.227107) (stroke (width 0.05) (type solid)) (layer "Edge.Cuts"))
 (gr_arc (start 170.442893 31.567107) (mid 171.15 31.86) (end 171.442893 32.567107) (stroke (width 0.05) (type solid)) (layer "Edge.Cuts"))
 (gr_line (start 152.827107 213.137106) (end 69.454583 213.241323) (stroke (width 0.05) (type solid)) (layer "Edge.Cuts"))
 (gr_line (start 75.755787 25.332892) (end 75.755787 24.832897) (stroke (width 0.05) (type solid)) (layer "Edge.Cuts"))
 (gr_line (start 29.723954 95.120516) (end 29.73 31.327108) (stroke (width 0.05) (type solid)) (layer "Edge.Cuts"))
 (gr_arc (start 132.192893 26.029094) (mid 132.9 26.321987) (end 133.192893 27.029094) (stroke (width 0.05) (type solid))
  (layer "Edge.Cuts"))
 (gr_arc (start 94.805787 22.832897) (mid 94.512894 23.540004) (end 93.805787 23.832897) (stroke (width 0.05) (type solid))
  (layer "Edge.Cuts"))
 (gr_line (start 95.805787 21.332897) (end 113.009993 21.332897) (stroke (width 0.05) (type solid)) (layer "Edge.Cuts"))
 (gr_arc (start 29.723954 95.120556) (mid 29.543054 95.694216) (end 29.065798 96.060313) (stroke (width 0.05) (type solid))
  (layer "Edge.Cuts"))
 (gr_line (start 37.474828 145.717107) (end 37.457107 167.56) (stroke (width 0.05) (type default)) (layer "Edge.Cuts"))
 (gr_line (start 172.02 194.092894) (end 154.8271 194.087107) (stroke (width 0.05) (type solid)) (layer "Edge.Cuts"))
 (gr_line (start 113.77 136.470242) (end 172.02 136.477106) (stroke (width 0.05) (type solid)) (layer "Edge.Cuts"))
 (gr_arc (start 173.02 193.1) (mid 172.727107 193.807107) (end 172.02 194.1) (stroke (width 0.05) (type solid)) (layer "Edge.Cuts"))
 (gr_line (start 171.442893 32.567107) (end 171.442893 88.190001) (stroke (width 0.05) (type solid)) (layer "Edge.Cuts"))
 (gr_arc (start 113.01 21.332897) (mid 113.717107 21.62579) (end 114.01 22.332897) (stroke (width 0.05) (type solid)) (layer "Edge.Cuts"))
 (gr_line (start 134.192893 31.560243) (end 170.442893 31.567107) (stroke (width 0.05) (type solid)) (layer "Edge.Cuts"))
 (gr_line (start 67.877382 108.329748) (end 48.768345 111.705734) (stroke (width 0.05) (type solid)) (layer "Edge.Cuts"))
 (gr_line (start 153.827107 195.087107) (end 153.827107 212.137106) (stroke (width 0.05) (type solid)) (layer "Edge.Cuts"))
 (gr_line (start 114.01 22.332897) (end 114.01 25.032897) (stroke (width 0.05) (type solid)) (layer "Edge.Cuts"))
 (gr_arc (start 79.42 184.472893) (mid 78.712893 184.18) (end 78.42 183.472893) (stroke (width 0.05) (type solid)) (layer "Edge.Cuts"))
 (gr_line (start 170.442893 89.182895) (end 153.249993 89.177108) (stroke (width 0.05) (type solid)) (layer "Edge.Cuts"))
 (gr_line (start 94.805787 22.832897) (end 94.805787 22.332897) (stroke (width 0.05) (type solid)) (layer "Edge.Cuts"))
 (gr_arc (start 172.02 136.477106) (mid 172.727107 136.769999) (end 173.02 137.477106) (stroke (width 0.05) (type solid))
  (layer "Edge.Cuts"))
 (gr_line (start 30.73 30.332893) (end 55.401695 30.332893) (stroke (width 0.05) (type solid)) (layer "Edge.Cuts"))
 (gr_arc (start 152.25 90.177108) (mid 152.542893 89.470001) (end 153.25 89.177108) (stroke (width 0.05) (type solid)) (layer "Edge.Cuts"))
 (gr_line (start 31.301061 200.030515) (end 31.307107 136.237107) (stroke (width 0.05) (type solid)) (layer "Edge.Cuts"))
 (gr_arc (start 75.755787 25.332892) (mid 75.462894 26.039999) (end 74.755787 26.332892) (stroke (width 0.05) (type solid))
  (layer "Edge.Cuts"))
 (gr_arc (start 31.301061 200.030555) (mid 31.120161 200.604215) (end 30.642905 200.970312) (stroke (width 0.05) (type solid))
  (layer "Edge.Cuts"))
 (gr_line (start 76.755787 23.832897) (end 93.805787 23.832897) (stroke (width 0.05) (type solid)) (layer "Edge.Cuts"))
 (gr_line (start 53.363508 145.717107) (end 53.345787 167.559999) (stroke (width 0.05) (type default)) (layer "Edge.Cuts"))
 (gr_arc (start 52.372893 144.717107) (mid 53.08 145.01) (end 53.372893 145.717107) (stroke (width 0.05) (type solid)) (layer "Edge.Cuts"))
 (gr_line (start 48.264907 111.840684) (end 32.02316 117.748752) (stroke (width 0.05) (type solid)) (layer "Edge.Cuts"))
 (gr_arc (start 153.827107 212.137106) (mid 153.534214 212.844213) (end 152.827107 213.137106) (stroke (width 0.05) (type solid))
  (layer "Edge.Cuts"))
 (gr_arc (start 112.762893 183.472893) (mid 112.47 184.18) (end 111.762893 184.472893) (stroke (width 0.05) (type solid))
  (layer "Edge.Cuts"))
 (gr_arc (start 31.307107 136.237107) (mid 31.6 135.53) (end 32.307107 135.237107) (stroke (width 0.05) (type solid)) (layer "Edge.Cuts"))
 (gr_line (start 69.454583 213.241323) (end 50.345452 216.615733) (stroke (width 0.05) (type solid)) (layer "Edge.Cuts"))
 (gr_arc (start 49.842013 216.750683) (mid 50.090796 216.672254) (end 50.345452 216.615733) (stroke (width 0.05) (type solid))
  (layer "Edge.Cuts"))
 (gr_line (start 78.43 136.240007) (end 78.42 183.472893) (stroke (width 0.05) (type default)) (layer "Edge.Cuts"))
 (gr_arc (start 56.407705 27.334809) (mid 56.699919 26.626463) (end 57.407703 26.332892) (stroke (width 0.05) (type solid))
  (layer "Edge.Cuts"))
 (gr_arc (start 48.264906 111.840684) (mid 48.513689 111.762255) (end 48.768345 111.705734) (stroke (width 0.05) (type solid))
  (layer "Edge.Cuts"))
 (gr_arc (start 152.25 107.227107) (mid 151.957107 107.934214) (end 151.25 108.227107) (stroke (width 0.05) (type solid))
  (layer "Edge.Cuts"))
 (gr_line (start 32.318666 222.060838) (end 25.692087 203.841601) (stroke (width 0.05) (type solid)) (layer "Edge.Cuts"))
 (gr_arc (start 134.192893 31.55622) (mid 133.485786 31.263327) (end 133.192893 30.55622) (stroke (width 0.05) (type solid))
  (layer "Edge.Cuts"))
 (gr_arc (start 94.805787 22.332897) (mid 95.09868 21.62579) (end 95.805787 21.332897) (stroke (width 0.05) (type solid))
  (layer "Edge.Cuts"))
 (gr_line (start 57.407703 26.332892) (end 74.755787 26.332892) (stroke (width 0.05) (type solid)) (layer "Edge.Cuts"))
 (gr_arc (start 53.345787 167.559999) (mid 53.052894 168.267106) (end 52.345787 168.559999) (stroke (width 0.05) (type solid))
  (layer "Edge.Cuts"))
 (gr_line (start 52.345787 168.559999) (end 38.4571 168.559999) (stroke (width 0.05) (type default)) (layer "Edge.Cuts"))
 (gr_arc (start 29.73 31.327108) (mid 30.022893 30.620001) (end 30.73 30.327108) (stroke (width 0.05) (type solid)) (layer "Edge.Cuts"))
 (gr_arc (start 24.11498 98.931602) (mid 24.148535 98.166982) (end 24.712893 97.650001) (stroke (width 0.05) (type solid))
  (layer "Edge.Cuts"))
 (gr_arc (start 75.755787 24.832897) (mid 76.04868 24.12579) (end 76.755787 23.832897) (stroke (width 0.05) (type solid))
  (layer "Edge.Cuts"))
 (gr_line (start 26.29 202.56) (end 30.642905 200.970312) (stroke (width 0.05) (type solid)) (layer "Edge.Cuts"))
 (gr_arc (start 56.411532 29.330975) (mid 56.119318 30.039321) (end 55.411534 30.332892) (stroke (width 0.05) (type solid))
  (layer "Edge.Cuts"))
 (gr_arc (start 32.02316 117.748752) (mid 31.258528 117.715224) (end 30.741559 117.150839) (stroke (width 0.05) (type solid))
  (layer "Edge.Cuts"))
 (gr_arc (start 25.692087 203.841601) (mid 25.725642 203.076981) (end 26.29 202.56) (stroke (width 0.05) (type solid)) (layer "Edge.Cuts"))
 (gr_arc (start 112.77 137.47) (mid 113.062893 136.762893) (end 113.77 136.47) (stroke (width 0.05) (type solid)) (layer "Edge.Cuts"))
 (gr_line (start 32.307107 135.242892) (end 77.43 135.240007) (stroke (width 0.05) (type solid)) (layer "Edge.Cuts"))
 (segment (start 43.752893 56.510001) (end 43.752893 55.260001) (width 0.5) (layer "B.Cu") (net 27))
 (segment (start 51.677893 46.150001) (end 51.662893 46.135001) (width 0.5) (layer "F.Cu") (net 14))
 (segment (start 36.382893 41.060001) (end 36.387893 41.055001) (width 0.5) (layer "F.Cu") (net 9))
 (segment (start 36.312893 38.590001) (end 36.387893 38.515001) (width 0.5) (layer "F.Cu") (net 5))
 (segment (start 51.662893 38.515001) (end 52.032455 38.515001) (width 0.5) (layer "F.Cu") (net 6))
 (segment (start 45.060601 46.830001) (end 45.041441 46.847541) (width 0.5) (layer "F.Cu") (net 3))
 (segment (start 36.382893 33.440001) (end 36.387893 33.435001) (width 0.5) (layer "F.Cu") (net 8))
 (segment (start 126.032893 89.920001) (end 126.022893 89.910001) (width 0.5) (layer "F.Cu") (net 4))
 (segment (start 36.382893 35.970001) (end 36.387893 35.975001) (width 0.5) (layer "F.Cu") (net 4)))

